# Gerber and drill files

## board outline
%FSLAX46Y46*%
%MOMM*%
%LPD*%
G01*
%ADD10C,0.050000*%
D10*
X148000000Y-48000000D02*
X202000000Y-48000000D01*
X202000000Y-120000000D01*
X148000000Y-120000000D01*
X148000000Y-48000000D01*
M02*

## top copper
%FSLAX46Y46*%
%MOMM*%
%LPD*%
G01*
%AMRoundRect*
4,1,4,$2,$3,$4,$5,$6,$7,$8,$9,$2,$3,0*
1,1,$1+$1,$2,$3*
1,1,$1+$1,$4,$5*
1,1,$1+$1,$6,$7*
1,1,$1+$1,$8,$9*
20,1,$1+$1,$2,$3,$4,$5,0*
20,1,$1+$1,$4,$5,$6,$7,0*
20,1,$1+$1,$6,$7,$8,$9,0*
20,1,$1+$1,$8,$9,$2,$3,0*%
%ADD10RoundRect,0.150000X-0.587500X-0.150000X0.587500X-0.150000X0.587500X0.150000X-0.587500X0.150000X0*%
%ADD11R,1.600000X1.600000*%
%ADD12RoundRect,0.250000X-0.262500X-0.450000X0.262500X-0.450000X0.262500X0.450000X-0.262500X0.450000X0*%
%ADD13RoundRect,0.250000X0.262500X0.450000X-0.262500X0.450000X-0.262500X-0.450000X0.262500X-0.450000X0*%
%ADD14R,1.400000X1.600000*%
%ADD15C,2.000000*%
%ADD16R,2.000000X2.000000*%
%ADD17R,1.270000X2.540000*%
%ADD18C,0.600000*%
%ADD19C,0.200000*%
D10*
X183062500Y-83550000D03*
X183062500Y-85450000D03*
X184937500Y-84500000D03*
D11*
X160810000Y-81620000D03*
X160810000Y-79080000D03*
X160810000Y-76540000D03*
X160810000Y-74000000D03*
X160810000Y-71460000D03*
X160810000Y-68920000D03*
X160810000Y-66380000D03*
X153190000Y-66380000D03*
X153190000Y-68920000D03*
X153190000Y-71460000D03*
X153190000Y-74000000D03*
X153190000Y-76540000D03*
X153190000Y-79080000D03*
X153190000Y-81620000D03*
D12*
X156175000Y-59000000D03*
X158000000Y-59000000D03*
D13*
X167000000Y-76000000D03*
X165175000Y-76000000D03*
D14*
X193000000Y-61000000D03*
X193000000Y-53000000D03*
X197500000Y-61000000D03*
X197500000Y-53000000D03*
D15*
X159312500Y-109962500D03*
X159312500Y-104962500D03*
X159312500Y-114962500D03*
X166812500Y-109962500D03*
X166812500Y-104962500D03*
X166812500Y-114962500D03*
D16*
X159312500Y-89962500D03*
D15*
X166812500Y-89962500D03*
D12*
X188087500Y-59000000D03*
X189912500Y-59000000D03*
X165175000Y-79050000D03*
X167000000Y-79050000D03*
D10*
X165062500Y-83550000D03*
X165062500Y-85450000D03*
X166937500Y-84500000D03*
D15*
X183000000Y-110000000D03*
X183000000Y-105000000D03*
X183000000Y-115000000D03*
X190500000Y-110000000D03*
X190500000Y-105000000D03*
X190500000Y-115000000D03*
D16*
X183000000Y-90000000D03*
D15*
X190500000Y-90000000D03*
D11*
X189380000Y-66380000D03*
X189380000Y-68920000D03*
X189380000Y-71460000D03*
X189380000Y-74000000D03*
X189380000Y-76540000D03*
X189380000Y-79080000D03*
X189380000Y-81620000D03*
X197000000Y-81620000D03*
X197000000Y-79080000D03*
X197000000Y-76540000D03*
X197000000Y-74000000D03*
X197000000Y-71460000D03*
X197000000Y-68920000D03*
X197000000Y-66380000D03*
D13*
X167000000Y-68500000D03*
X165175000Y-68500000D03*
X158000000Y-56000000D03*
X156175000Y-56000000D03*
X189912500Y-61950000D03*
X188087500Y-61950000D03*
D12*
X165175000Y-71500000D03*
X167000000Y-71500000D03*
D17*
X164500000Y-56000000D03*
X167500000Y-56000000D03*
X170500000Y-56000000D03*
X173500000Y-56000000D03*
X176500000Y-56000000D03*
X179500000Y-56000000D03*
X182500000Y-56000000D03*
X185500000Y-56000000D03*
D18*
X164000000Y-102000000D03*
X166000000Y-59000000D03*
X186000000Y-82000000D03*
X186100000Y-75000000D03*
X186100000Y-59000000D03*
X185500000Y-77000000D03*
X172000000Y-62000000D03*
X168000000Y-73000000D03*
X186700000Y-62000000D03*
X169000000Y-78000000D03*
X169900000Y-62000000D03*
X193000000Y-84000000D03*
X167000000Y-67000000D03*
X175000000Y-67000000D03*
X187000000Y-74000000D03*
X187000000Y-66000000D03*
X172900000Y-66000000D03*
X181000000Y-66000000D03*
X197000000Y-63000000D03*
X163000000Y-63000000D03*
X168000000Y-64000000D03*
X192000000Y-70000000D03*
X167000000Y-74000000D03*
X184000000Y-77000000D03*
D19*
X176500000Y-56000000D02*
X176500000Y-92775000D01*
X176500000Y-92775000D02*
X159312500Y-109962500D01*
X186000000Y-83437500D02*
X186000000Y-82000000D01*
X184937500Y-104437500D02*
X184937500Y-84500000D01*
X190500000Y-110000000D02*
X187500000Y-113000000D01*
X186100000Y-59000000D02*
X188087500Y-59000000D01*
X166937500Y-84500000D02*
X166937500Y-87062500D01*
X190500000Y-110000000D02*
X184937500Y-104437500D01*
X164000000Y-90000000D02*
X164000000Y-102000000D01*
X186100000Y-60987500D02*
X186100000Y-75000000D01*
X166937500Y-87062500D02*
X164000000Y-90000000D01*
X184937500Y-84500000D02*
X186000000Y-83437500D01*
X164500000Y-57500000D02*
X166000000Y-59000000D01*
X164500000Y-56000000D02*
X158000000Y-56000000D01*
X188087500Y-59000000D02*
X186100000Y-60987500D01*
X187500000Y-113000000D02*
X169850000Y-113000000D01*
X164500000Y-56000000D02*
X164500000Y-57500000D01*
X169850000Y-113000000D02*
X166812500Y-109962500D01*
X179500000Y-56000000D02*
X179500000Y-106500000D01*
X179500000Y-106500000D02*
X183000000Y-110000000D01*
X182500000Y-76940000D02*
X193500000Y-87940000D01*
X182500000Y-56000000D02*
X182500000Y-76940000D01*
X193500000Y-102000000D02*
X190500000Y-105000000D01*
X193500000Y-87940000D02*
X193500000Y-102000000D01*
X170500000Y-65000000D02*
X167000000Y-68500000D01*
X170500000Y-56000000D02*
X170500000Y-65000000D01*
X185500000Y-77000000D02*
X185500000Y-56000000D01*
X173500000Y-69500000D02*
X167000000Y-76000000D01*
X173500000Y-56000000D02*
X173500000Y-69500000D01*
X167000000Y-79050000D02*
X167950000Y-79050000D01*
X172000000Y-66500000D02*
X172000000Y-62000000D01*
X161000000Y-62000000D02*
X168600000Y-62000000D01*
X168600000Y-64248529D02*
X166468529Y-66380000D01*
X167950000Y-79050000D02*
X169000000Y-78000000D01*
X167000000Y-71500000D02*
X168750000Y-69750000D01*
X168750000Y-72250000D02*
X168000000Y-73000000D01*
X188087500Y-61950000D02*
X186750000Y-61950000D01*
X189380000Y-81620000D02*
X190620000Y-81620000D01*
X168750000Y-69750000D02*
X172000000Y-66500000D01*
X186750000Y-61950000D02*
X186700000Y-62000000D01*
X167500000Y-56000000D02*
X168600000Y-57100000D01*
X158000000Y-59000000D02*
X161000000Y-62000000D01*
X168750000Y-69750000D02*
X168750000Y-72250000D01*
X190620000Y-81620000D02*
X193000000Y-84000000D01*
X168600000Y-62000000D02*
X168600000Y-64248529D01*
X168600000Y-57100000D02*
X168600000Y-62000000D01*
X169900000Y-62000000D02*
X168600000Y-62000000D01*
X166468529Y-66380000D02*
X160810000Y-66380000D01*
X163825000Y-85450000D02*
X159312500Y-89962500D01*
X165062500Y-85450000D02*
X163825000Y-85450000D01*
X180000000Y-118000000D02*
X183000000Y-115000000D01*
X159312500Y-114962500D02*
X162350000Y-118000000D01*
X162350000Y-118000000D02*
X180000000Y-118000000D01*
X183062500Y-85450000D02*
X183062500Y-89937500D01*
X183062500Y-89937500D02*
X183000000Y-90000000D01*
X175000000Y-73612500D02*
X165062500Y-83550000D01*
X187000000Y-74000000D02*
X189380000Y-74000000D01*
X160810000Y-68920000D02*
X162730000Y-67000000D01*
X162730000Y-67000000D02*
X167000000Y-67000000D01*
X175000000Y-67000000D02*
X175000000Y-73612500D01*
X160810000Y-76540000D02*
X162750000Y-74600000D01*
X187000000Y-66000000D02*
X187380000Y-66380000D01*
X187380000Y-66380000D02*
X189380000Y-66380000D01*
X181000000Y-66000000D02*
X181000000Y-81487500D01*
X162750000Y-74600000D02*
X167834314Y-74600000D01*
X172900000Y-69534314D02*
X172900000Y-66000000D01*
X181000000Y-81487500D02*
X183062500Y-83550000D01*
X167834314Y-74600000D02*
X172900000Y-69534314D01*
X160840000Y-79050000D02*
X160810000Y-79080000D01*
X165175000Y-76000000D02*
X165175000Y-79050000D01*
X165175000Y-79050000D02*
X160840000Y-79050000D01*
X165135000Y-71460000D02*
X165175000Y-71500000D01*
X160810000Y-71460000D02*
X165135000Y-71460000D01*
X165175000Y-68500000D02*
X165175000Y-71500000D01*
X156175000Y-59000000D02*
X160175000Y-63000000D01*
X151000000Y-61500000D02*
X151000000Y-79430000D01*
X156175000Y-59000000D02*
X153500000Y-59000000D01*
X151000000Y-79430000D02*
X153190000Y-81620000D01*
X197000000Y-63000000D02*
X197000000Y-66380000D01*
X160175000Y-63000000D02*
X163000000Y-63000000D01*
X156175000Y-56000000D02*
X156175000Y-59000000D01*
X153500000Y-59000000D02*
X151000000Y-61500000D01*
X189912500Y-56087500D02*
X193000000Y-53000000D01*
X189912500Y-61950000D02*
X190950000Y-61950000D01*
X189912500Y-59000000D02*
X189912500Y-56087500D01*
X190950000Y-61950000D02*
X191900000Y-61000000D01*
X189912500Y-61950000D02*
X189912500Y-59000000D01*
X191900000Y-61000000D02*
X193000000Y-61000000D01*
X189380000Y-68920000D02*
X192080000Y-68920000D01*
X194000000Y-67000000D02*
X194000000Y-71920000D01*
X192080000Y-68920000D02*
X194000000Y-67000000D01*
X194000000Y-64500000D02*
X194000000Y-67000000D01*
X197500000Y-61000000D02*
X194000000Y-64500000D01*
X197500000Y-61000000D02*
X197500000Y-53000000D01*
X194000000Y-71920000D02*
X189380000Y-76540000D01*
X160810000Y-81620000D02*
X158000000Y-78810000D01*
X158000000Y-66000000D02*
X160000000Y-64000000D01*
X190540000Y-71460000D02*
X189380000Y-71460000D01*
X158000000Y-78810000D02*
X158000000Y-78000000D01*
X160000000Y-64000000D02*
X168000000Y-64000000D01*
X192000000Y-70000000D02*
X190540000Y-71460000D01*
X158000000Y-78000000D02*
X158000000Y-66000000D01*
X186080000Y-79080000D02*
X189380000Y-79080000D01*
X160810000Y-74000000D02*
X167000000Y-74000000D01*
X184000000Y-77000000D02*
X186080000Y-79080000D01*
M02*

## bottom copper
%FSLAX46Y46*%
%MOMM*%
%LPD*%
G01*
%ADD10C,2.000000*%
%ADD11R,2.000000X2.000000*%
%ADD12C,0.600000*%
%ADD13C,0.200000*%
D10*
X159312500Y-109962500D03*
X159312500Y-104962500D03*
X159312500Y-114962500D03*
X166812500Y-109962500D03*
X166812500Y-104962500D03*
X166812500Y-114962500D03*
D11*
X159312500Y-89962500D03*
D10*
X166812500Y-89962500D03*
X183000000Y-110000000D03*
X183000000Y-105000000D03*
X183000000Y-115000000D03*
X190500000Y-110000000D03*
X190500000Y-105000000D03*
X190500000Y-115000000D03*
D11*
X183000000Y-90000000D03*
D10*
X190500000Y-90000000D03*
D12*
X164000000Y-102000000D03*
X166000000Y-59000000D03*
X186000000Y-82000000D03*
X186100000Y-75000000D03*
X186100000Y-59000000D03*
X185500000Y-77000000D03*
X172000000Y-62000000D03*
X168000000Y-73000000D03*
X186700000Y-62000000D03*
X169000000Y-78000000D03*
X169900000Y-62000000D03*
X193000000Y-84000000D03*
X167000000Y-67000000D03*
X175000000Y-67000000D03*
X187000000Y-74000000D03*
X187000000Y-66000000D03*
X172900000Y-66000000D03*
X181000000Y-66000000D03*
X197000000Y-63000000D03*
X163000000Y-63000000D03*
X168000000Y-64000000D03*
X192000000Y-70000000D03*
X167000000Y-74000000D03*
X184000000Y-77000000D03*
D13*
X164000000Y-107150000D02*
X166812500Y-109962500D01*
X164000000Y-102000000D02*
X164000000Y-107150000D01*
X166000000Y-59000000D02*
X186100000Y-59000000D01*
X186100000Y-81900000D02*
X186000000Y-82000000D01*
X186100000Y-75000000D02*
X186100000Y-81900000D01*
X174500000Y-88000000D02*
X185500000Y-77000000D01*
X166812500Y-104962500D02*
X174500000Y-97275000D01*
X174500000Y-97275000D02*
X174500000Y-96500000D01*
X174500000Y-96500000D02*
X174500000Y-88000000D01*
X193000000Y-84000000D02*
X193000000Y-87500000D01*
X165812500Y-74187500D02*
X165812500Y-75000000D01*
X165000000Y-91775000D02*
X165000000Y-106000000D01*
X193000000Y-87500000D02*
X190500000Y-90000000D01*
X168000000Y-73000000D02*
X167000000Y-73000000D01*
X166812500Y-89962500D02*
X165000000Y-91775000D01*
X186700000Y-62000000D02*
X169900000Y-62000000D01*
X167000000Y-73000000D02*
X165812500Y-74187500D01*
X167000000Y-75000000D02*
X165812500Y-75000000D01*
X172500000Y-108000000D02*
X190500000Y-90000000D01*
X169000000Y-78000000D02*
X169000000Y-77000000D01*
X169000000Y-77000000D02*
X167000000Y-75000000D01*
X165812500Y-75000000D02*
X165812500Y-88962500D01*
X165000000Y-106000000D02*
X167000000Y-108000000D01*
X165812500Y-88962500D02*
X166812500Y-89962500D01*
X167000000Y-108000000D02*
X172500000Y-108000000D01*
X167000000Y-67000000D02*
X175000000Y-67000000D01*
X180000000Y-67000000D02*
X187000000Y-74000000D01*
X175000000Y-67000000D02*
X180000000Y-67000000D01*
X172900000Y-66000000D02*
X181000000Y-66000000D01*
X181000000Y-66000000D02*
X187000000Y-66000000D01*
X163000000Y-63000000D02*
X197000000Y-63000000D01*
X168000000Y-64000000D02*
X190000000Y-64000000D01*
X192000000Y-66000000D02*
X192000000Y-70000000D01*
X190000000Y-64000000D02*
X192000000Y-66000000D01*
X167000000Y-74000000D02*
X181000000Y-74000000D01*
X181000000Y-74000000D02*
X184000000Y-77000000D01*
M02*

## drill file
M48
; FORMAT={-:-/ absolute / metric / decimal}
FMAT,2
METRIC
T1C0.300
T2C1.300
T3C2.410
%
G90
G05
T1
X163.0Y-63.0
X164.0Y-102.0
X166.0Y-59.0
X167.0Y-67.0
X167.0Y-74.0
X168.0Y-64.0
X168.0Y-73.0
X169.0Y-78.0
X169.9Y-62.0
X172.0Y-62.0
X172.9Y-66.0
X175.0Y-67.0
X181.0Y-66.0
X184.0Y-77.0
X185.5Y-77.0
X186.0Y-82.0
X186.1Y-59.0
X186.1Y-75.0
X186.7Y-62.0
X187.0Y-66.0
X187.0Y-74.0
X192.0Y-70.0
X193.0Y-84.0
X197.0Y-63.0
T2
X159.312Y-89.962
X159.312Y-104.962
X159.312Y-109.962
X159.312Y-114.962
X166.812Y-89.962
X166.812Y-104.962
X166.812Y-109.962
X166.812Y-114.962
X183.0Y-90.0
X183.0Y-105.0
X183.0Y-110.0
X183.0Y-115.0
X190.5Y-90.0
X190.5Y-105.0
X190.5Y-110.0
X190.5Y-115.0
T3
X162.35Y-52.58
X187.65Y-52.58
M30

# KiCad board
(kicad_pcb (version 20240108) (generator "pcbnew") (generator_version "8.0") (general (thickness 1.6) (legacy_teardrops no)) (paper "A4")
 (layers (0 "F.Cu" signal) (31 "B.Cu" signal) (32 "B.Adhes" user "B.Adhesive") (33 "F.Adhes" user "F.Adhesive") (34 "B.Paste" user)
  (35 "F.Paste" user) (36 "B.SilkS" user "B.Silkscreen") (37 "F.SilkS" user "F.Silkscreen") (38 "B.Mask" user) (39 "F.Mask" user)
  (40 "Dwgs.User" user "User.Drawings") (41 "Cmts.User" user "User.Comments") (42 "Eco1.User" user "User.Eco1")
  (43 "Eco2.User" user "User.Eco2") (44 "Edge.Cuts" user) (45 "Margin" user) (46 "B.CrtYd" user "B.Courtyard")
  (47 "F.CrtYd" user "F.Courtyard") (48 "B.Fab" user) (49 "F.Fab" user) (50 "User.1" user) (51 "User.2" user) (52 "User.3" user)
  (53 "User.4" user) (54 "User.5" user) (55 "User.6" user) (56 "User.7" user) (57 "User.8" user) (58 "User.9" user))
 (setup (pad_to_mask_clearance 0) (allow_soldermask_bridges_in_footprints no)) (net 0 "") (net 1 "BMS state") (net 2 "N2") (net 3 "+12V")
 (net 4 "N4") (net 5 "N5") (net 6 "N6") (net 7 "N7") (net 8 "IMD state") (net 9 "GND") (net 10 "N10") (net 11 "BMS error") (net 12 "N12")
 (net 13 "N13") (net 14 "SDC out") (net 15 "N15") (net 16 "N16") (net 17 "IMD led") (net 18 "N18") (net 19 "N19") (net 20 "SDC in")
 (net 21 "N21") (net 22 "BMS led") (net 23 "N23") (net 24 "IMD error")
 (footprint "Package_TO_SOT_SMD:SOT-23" (layer "F.Cu") (at 184 84.5)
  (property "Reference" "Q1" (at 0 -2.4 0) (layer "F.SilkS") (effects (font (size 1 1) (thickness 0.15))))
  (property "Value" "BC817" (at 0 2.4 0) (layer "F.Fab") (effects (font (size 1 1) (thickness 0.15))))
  (pad "1" smd roundrect (at -0.9375 -0.95) (size 1.475 0.6) (layers "F.Cu" "F.Paste" "F.Mask") (roundrect_rratio 0.25) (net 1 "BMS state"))
  (pad "2" smd roundrect (at -0.9375 0.95) (size 1.475 0.6) (layers "F.Cu" "F.Paste" "F.Mask") (roundrect_rratio 0.25) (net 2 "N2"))
  (pad "3" smd roundrect (at 0.9375 0) (size 1.475 0.6) (layers "F.Cu" "F.Paste" "F.Mask") (roundrect_rratio 0.25) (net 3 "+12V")))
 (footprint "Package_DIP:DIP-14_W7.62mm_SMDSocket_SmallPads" (layer "F.Cu") (at 157 74 180)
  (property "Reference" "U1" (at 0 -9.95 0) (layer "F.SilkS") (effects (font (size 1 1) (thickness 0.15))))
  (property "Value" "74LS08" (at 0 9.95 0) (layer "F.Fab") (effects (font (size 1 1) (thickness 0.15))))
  (pad "1" smd rect (at -3.81 -7.62 180) (size 1.6 1.6) (layers "F.Cu" "F.Paste" "F.Mask") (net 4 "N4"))
  (pad "2" smd rect (at -3.81 -5.08 180) (size 1.6 1.6) (layers "F.Cu" "F.Paste" "F.Mask") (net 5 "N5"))
  (pad "3" smd rect (at -3.81 -2.54 180) (size 1.6 1.6) (layers "F.Cu" "F.Paste" "F.Mask") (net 1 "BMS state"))
  (pad "4" smd rect (at -3.81 0 180) (size 1.6 1.6) (layers "F.Cu" "F.Paste" "F.Mask") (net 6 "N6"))
  (pad "5" smd rect (at -3.81 2.54 180) (size 1.6 1.6) (layers "F.Cu" "F.Paste" "F.Mask") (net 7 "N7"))
  (pad "6" smd rect (at -3.81 5.08 180) (size 1.6 1.6) (layers "F.Cu" "F.Paste" "F.Mask") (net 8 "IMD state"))
  (pad "7" smd rect (at -3.81 7.62 180) (size 1.6 1.6) (layers "F.Cu" "F.Paste" "F.Mask") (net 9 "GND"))
  (pad "8" smd rect (at 3.81 7.62 180) (size 1.6 1.6) (layers "F.Cu" "F.Paste" "F.Mask"))
  (pad "9" smd rect (at 3.81 5.08 180) (size 1.6 1.6) (layers "F.Cu" "F.Paste" "F.Mask"))
  (pad "10" smd rect (at 3.81 2.54 180) (size 1.6 1.6) (layers "F.Cu" "F.Paste" "F.Mask"))
  (pad "11" smd rect (at 3.81 0 180) (size 1.6 1.6) (layers "F.Cu" "F.Paste" "F.Mask"))
  (pad "12" smd rect (at 3.81 -2.54 180) (size 1.6 1.6) (layers "F.Cu" "F.Paste" "F.Mask"))
  (pad "13" smd rect (at 3.81 -5.08 180) (size 1.6 1.6) (layers "F.Cu" "F.Paste" "F.Mask"))
  (pad "14" smd rect (at 3.81 -7.62 180) (size 1.6 1.6) (layers "F.Cu" "F.Paste" "F.Mask") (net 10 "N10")))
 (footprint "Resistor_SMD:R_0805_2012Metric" (layer "F.Cu") (at 157.0875 59)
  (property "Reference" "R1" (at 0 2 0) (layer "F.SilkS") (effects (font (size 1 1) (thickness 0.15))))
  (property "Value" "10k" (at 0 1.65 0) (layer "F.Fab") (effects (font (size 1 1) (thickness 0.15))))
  (pad "1" smd roundrect (at -0.9125 0) (size 1.025 1.4) (layers "F.Cu" "F.Paste" "F.Mask") (roundrect_rratio 0.243902) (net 10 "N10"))
  (pad "2" smd roundrect (at 0.9125 0) (size 1.025 1.4) (layers "F.Cu" "F.Paste" "F.Mask") (roundrect_rratio 0.243902) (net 9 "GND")))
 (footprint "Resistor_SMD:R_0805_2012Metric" (layer "F.Cu") (at 166.0875 76 180)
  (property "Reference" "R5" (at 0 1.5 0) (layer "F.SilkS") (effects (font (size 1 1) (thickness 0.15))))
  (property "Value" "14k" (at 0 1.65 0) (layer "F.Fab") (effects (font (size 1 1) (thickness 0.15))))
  (pad "1" smd roundrect (at -0.9125 0 180) (size 1.025 1.4) (layers "F.Cu" "F.Paste" "F.Mask") (roundrect_rratio 0.243902)
   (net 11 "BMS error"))
  (pad "2" smd roundrect (at 0.9125 0 180) (size 1.025 1.4) (layers "F.Cu" "F.Paste" "F.Mask") (roundrect_rratio 0.243902) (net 5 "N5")))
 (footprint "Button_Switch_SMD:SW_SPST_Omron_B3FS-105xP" (layer "F.Cu") (at 195.25 57 90)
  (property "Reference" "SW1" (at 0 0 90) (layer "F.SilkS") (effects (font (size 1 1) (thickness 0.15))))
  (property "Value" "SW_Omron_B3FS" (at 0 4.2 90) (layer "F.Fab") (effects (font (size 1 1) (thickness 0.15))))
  (pad "1" smd rect (at -4 -2.25 270) (size 1.6 1.4) (layers "F.Cu" "F.Paste" "F.Mask") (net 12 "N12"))
  (pad "1" smd rect (at 4 -2.25 270) (size 1.6 1.4) (layers "F.Cu" "F.Paste" "F.Mask") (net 12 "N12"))
  (pad "2" smd rect (at -4 2.25 270) (size 1.6 1.4) (layers "F.Cu" "F.Paste" "F.Mask") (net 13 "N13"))
  (pad "2" smd rect (at 4 2.25 270) (size 1.6 1.4) (layers "F.Cu" "F.Paste" "F.Mask") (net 13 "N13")))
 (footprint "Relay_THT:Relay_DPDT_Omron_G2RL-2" (layer "F.Cu") (at 159.3125 89.9625)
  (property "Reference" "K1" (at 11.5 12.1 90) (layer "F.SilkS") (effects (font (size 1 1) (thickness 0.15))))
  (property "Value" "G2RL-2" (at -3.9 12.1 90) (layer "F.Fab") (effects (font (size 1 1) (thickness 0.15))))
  (pad "11" thru_hole circle (at 0 20) (size 2 2) (drill 1.3) (layers "*.Cu" "*.Mask") (remove_unused_layers no) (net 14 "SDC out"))
  (pad "12" thru_hole circle (at 0 15) (size 2 2) (drill 1.3) (layers "*.Cu" "*.Mask") (remove_unused_layers no) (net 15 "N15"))
  (pad "14" thru_hole circle (at 0 25) (size 2 2) (drill 1.3) (layers "*.Cu" "*.Mask") (remove_unused_layers no) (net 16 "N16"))
  (pad "21" thru_hole circle (at 7.5 20) (size 2 2) (drill 1.3) (layers "*.Cu" "*.Mask") (remove_unused_layers no) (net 3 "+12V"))
  (pad "22" thru_hole circle (at 7.5 15) (size 2 2) (drill 1.3) (layers "*.Cu" "*.Mask") (remove_unused_layers no) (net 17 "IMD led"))
  (pad "24" thru_hole circle (at 7.5 25) (size 2 2) (drill 1.3) (layers "*.Cu" "*.Mask") (remove_unused_layers no) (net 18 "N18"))
  (pad "A1" thru_hole rect (at 0 0) (size 2 2) (drill 1.3) (layers "*.Cu" "*.Mask") (remove_unused_layers no) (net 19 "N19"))
  (pad "A2" thru_hole circle (at 7.5 0) (size 2 2) (drill 1.3) (layers "*.Cu" "*.Mask") (remove_unused_layers no) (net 9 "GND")))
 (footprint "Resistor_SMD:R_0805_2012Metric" (layer "F.Cu") (at 189 59)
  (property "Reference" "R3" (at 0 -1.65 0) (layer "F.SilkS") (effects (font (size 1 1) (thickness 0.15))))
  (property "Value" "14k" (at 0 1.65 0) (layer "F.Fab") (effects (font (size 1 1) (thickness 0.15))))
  (pad "1" smd roundrect (at -0.9125 0) (size 1.025 1.4) (layers "F.Cu" "F.Paste" "F.Mask") (roundrect_rratio 0.243902) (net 3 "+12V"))
  (pad "2" smd roundrect (at 0.9125 0) (size 1.025 1.4) (layers "F.Cu" "F.Paste" "F.Mask") (roundrect_rratio 0.243902) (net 12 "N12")))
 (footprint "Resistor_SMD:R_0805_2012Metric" (layer "F.Cu") (at 166.0875 79.05)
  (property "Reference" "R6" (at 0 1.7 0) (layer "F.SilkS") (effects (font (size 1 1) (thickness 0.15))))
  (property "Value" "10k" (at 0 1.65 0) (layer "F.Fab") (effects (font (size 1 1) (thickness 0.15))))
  (pad "1" smd roundrect (at -0.9125 0) (size 1.025 1.4) (layers "F.Cu" "F.Paste" "F.Mask") (roundrect_rratio 0.243902) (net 5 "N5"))
  (pad "2" smd roundrect (at 0.9125 0) (size 1.025 1.4) (layers "F.Cu" "F.Paste" "F.Mask") (roundrect_rratio 0.243902) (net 9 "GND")))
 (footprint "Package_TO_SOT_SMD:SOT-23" (layer "F.Cu") (at 166 84.5)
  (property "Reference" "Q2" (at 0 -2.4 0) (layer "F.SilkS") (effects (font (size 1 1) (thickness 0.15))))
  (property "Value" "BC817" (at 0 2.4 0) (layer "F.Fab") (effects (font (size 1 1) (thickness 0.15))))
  (pad "1" smd roundrect (at -0.9375 -0.95) (size 1.475 0.6) (layers "F.Cu" "F.Paste" "F.Mask") (roundrect_rratio 0.25) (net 8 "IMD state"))
  (pad "2" smd roundrect (at -0.9375 0.95) (size 1.475 0.6) (layers "F.Cu" "F.Paste" "F.Mask") (roundrect_rratio 0.25) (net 19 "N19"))
  (pad "3" smd roundrect (at 0.9375 0) (size 1.475 0.6) (layers "F.Cu" "F.Paste" "F.Mask") (roundrect_rratio 0.25) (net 3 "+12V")))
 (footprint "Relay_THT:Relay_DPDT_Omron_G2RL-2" (layer "F.Cu") (at 183 90)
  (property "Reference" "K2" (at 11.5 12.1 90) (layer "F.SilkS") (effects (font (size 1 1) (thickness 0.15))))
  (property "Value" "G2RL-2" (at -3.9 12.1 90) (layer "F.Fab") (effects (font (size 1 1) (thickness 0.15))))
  (pad "11" thru_hole circle (at 0 20) (size 2 2) (drill 1.3) (layers "*.Cu" "*.Mask") (remove_unused_layers no) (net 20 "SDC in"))
  (pad "12" thru_hole circle (at 0 15) (size 2 2) (drill 1.3) (layers "*.Cu" "*.Mask") (remove_unused_layers no) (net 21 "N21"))
  (pad "14" thru_hole circle (at 0 25) (size 2 2) (drill 1.3) (layers "*.Cu" "*.Mask") (remove_unused_layers no) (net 16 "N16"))
  (pad "21" thru_hole circle (at 7.5 20) (size 2 2) (drill 1.3) (layers "*.Cu" "*.Mask") (remove_unused_layers no) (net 3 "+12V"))
  (pad "22" thru_hole circle (at 7.5 15) (size 2 2) (drill 1.3) (layers "*.Cu" "*.Mask") (remove_unused_layers no) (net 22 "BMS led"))
  (pad "24" thru_hole circle (at 7.5 25) (size 2 2) (drill 1.3) (layers "*.Cu" "*.Mask") (remove_unused_layers no) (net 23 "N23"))
  (pad "A1" thru_hole rect (at 0 0) (size 2 2) (drill 1.3) (layers "*.Cu" "*.Mask") (remove_unused_layers no) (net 2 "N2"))
  (pad "A2" thru_hole circle (at 7.5 0) (size 2 2) (drill 1.3) (layers "*.Cu" "*.Mask") (remove_unused_layers no) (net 9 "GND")))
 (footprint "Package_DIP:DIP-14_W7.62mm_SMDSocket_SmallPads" (layer "F.Cu") (at 193.19 74)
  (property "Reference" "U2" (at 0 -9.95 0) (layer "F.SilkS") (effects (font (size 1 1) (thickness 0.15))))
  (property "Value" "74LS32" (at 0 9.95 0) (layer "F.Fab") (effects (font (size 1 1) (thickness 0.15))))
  (pad "1" smd rect (at -3.81 -7.62) (size 1.6 1.6) (layers "F.Cu" "F.Paste" "F.Mask") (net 1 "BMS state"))
  (pad "2" smd rect (at -3.81 -5.08) (size 1.6 1.6) (layers "F.Cu" "F.Paste" "F.Mask") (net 13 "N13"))
  (pad "3" smd rect (at -3.81 -2.54) (size 1.6 1.6) (layers "F.Cu" "F.Paste" "F.Mask") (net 4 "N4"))
  (pad "4" smd rect (at -3.81 0) (size 1.6 1.6) (layers "F.Cu" "F.Paste" "F.Mask") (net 8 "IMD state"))
  (pad "5" smd rect (at -3.81 2.54) (size 1.6 1.6) (layers "F.Cu" "F.Paste" "F.Mask") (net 13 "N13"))
  (pad "6" smd rect (at -3.81 5.08) (size 1.6 1.6) (layers "F.Cu" "F.Paste" "F.Mask") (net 6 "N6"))
  (pad "7" smd rect (at -3.81 7.62) (size 1.6 1.6) (layers "F.Cu" "F.Paste" "F.Mask") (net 9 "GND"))
  (pad "8" smd rect (at 3.81 7.62) (size 1.6 1.6) (layers "F.Cu" "F.Paste" "F.Mask"))
  (pad "9" smd rect (at 3.81 5.08) (size 1.6 1.6) (layers "F.Cu" "F.Paste" "F.Mask"))
  (pad "10" smd rect (at 3.81 2.54) (size 1.6 1.6) (layers "F.Cu" "F.Paste" "F.Mask"))
  (pad "11" smd rect (at 3.81 0) (size 1.6 1.6) (layers "F.Cu" "F.Paste" "F.Mask"))
  (pad "12" smd rect (at 3.81 -2.54) (size 1.6 1.6) (layers "F.Cu" "F.Paste" "F.Mask"))
  (pad "13" smd rect (at 3.81 -5.08) (size 1.6 1.6) (layers "F.Cu" "F.Paste" "F.Mask"))
  (pad "14" smd rect (at 3.81 -7.62) (size 1.6 1.6) (layers "F.Cu" "F.Paste" "F.Mask") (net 10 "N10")))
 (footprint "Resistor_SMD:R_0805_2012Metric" (layer "F.Cu") (at 166.0875 68.5 180)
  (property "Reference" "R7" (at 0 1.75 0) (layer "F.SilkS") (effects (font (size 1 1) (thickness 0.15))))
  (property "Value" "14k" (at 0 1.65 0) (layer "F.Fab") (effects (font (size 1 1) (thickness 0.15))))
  (pad "1" smd roundrect (at -0.9125 0 180) (size 1.025 1.4) (layers "F.Cu" "F.Paste" "F.Mask") (roundrect_rratio 0.243902)
   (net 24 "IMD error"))
  (pad "2" smd roundrect (at 0.9125 0 180) (size 1.025 1.4) (layers "F.Cu" "F.Paste" "F.Mask") (roundrect_rratio 0.243902) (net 7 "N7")))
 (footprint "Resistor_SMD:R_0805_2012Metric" (layer "F.Cu") (at 157.0875 56 180)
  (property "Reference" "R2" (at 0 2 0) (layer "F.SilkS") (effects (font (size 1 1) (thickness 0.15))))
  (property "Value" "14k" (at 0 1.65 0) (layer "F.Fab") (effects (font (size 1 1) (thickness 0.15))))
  (pad "1" smd roundrect (at -0.9125 0 180) (size 1.025 1.4) (layers "F.Cu" "F.Paste" "F.Mask") (roundrect_rratio 0.243902) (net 3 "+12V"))
  (pad "2" smd roundrect (at 0.9125 0 180) (size 1.025 1.4) (layers "F.Cu" "F.Paste" "F.Mask") (roundrect_rratio 0.243902) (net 10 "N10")))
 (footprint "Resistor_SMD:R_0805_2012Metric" (layer "F.Cu") (at 189 61.95 180)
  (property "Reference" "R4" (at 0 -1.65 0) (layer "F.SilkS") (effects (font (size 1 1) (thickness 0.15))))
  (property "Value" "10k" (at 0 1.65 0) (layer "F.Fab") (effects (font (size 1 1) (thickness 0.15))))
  (pad "1" smd roundrect (at -0.9125 0 180) (size 1.025 1.4) (layers "F.Cu" "F.Paste" "F.Mask") (roundrect_rratio 0.243902) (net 12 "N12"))
  (pad "2" smd roundrect (at 0.9125 0 180) (size 1.025 1.4) (layers "F.Cu" "F.Paste" "F.Mask") (roundrect_rratio 0.243902) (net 9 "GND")))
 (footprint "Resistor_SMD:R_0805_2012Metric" (layer "F.Cu") (at 166.0875 71.5)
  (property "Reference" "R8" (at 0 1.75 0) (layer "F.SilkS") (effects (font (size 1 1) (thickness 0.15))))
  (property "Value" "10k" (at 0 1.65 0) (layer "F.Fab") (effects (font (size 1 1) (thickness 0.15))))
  (pad "1" smd roundrect (at -0.9125 0) (size 1.025 1.4) (layers "F.Cu" "F.Paste" "F.Mask") (roundrect_rratio 0.243902) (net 7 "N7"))
  (pad "2" smd roundrect (at 0.9125 0) (size 1.025 1.4) (layers "F.Cu" "F.Paste" "F.Mask") (roundrect_rratio 0.243902) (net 9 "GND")))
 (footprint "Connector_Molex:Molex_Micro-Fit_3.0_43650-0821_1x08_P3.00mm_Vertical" (layer "F.Cu") (at 175 52.865)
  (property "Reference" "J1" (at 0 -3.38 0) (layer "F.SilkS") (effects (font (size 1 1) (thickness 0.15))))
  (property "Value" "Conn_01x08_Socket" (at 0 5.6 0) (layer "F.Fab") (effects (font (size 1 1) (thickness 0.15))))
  (pad "" np_thru_hole circle (at -12.65 -0.285) (size 2.41 2.41) (drill 2.41) (layers "*.Cu" "*.Mask"))
  (pad "" np_thru_hole circle (at 12.65 -0.285) (size 2.41 2.41) (drill 2.41) (layers "*.Cu" "*.Mask"))
  (pad "1" smd rect (at -10.5 3.135) (size 1.27 2.54) (layers "F.Cu" "F.Paste" "F.Mask") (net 3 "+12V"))
  (pad "2" smd rect (at -7.5 3.135) (size 1.27 2.54) (layers "F.Cu" "F.Paste" "F.Mask") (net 9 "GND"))
  (pad "3" smd rect (at -4.5 3.135) (size 1.27 2.54) (layers "F.Cu" "F.Paste" "F.Mask") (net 24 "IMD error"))
  (pad "4" smd rect (at -1.5 3.135) (size 1.27 2.54) (layers "F.Cu" "F.Paste" "F.Mask") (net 11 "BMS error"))
  (pad "5" smd rect (at 1.5 3.135) (size 1.27 2.54) (layers "F.Cu" "F.Paste" "F.Mask") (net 14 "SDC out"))
  (pad "6" smd rect (at 4.5 3.135) (size 1.27 2.54) (layers "F.Cu" "F.Paste" "F.Mask") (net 20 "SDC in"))
  (pad "7" smd rect (at 7.5 3.135) (size 1.27 2.54) (layers "F.Cu" "F.Paste" "F.Mask") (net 22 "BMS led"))
  (pad "8" smd rect (at 10.5 3.135) (size 1.27 2.54) (layers "F.Cu" "F.Paste" "F.Mask") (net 17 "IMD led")))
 (gr_rect (start 148 48) (end 202 120) (stroke (width 0.05) (type default)) (fill none) (layer "Edge.Cuts"))
 (segment (start 176.5 56) (end 176.5 92.775) (width 0.2) (layer "F.Cu") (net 14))
 (segment (start 176.5 92.775) (end 159.3125 109.9625) (width 0.2) (layer "F.Cu") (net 14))
 (segment (start 186 83.4375) (end 186 82) (width 0.2) (layer "F.Cu") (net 3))
 (segment (start 184.9375 104.4375) (end 184.9375 84.5) (width 0.2) (layer "F.Cu") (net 3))
 (segment (start 190.5 110) (end 187.5 113) (width 0.2) (layer "F.Cu") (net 3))
 (segment (start 186.1 59) (end 188.0875 59) (width 0.2) (layer "F.Cu") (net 3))
 (segment (start 166.9375 84.5) (end 166.9375 87.0625) (width 0.2) (layer "F.Cu") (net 3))
 (segment (start 190.5 110) (end 184.9375 104.4375) (width 0.2) (layer "F.Cu") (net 3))
 (segment (start 164 90) (end 164 102) (width 0.2) (layer "F.Cu") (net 3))
 (segment (start 186.1 60.9875) (end 186.1 75) (width 0.2) (layer "F.Cu") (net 3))
 (segment (start 166.9375 87.0625) (end 164 90) (width 0.2) (layer "F.Cu") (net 3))
 (segment (start 184.9375 84.5) (end 186 83.4375) (width 0.2) (layer "F.Cu") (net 3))
 (segment (start 164.5 57.5) (end 166 59) (width 0.2) (layer "F.Cu") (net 3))
 (segment (start 164.5 56) (end 158 56) (width 0.2) (layer "F.Cu") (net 3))
 (segment (start 188.0875 59) (end 186.1 60.9875) (width 0.2) (layer "F.Cu") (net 3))
 (segment (start 187.5 113) (end 169.85 113) (width 0.2) (layer "F.Cu") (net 3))
 (segment (start 164.5 56) (end 164.5 57.5) (width 0.2) (layer "F.Cu") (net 3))
 (segment (start 169.85 113) (end 166.8125 109.9625) (width 0.2) (layer "F.Cu") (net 3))
 (via (at 164 102) (size 0.6) (drill 0.3) (layers "F.Cu" "B.Cu") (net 3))
 (via (at 166 59) (size 0.6) (drill 0.3) (layers "F.Cu" "B.Cu") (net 3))
 (via (at 186 82) (size 0.6) (drill 0.3) (layers "F.Cu" "B.Cu") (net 3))
 (via (at 186.1 75) (size 0.6) (drill 0.3) (layers "F.Cu" "B.Cu") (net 3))
 (via (at 186.1 59) (size 0.6) (drill 0.3) (layers "F.Cu" "B.Cu") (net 3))
 (segment (start 164 107.15) (end 166.8125 109.9625) (width 0.2) (layer "B.Cu") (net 3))
 (segment (start 164 102) (end 164 107.15) (width 0.2) (layer "B.Cu") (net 3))
 (segment (start 166 59) (end 186.1 59) (width 0.2) (layer "B.Cu") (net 3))
 (segment (start 186.1 81.9) (end 186 82) (width 0.2) (layer "B.Cu") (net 3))
 (segment (start 186.1 75) (end 186.1 81.9) (width 0.2) (layer "B.Cu") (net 3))
 (segment (start 179.5 56) (end 179.5 106.5) (width 0.2) (layer "F.Cu") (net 20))
 (segment (start 179.5 106.5) (end 183 110) (width 0.2) (layer "F.Cu") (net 20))
 (segment (start 182.5 76.94) (end 193.5 87.94) (width 0.2) (layer "F.Cu") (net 22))
 (segment (start 182.5 56) (end 182.5 76.94) (width 0.2) (layer "F.Cu") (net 22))
 (segment (start 193.5 102) (end 190.5 105) (width 0.2) (layer "F.Cu") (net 22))
 (segment (start 193.5 87.94) (end 193.5 102) (width 0.2) (layer "F.Cu") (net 22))
 (segment (start 170.5 65) (end 167 68.5) (width 0.2) (layer "F.Cu") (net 24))
 (segment (start 170.5 56) (end 170.5 65) (width 0.2) (layer "F.Cu") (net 24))
 (segment (start 185.5 77) (end 185.5 56) (width 0.2) (layer "F.Cu") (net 17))
 (via (at 185.5 77) (size 0.6) (drill 0.3) (layers "F.Cu" "B.Cu") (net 17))
 (segment (start 174.5 88) (end 185.5 77) (width 0.2) (layer "B.Cu") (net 17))
 (segment (start 166.8125 104.9625) (end 174.5 97.275) (width 0.2) (layer "B.Cu") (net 17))
 (segment (start 174.5 97.275) (end 174.5 96.5) (width 0.2) (layer "B.Cu") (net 17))
 (segment (start 174.5 96.5) (end 174.5 88) (width 0.2) (layer "B.Cu") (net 17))
 (segment (start 173.5 69.5) (end 167 76) (width 0.2) (layer "F.Cu") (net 11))
 (segment (start 173.5 56) (end 173.5 69.5) (width 0.2) (layer "F.Cu") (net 11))
 (segment (start 167 79.05) (end 167.95 79.05) (width 0.2) (layer "F.Cu") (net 9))
 (segment (start 172 66.5) (end 172 62) (width 0.2) (layer "F.Cu") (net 9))
 (segment (start 161 62) (end 168.6 62) (width 0.2) (layer "F.Cu") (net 9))
 (segment (start 168.6 64.248529) (end 166.468529 66.38) (width 0.2) (layer "F.Cu") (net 9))
 (segment (start 167.95 79.05) (end 169 78) (width 0.2) (layer "F.Cu") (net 9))
 (segment (start 167 71.5) (end 168.75 69.75) (width 0.2) (layer "F.Cu") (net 9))
 (segment (start 168.75 72.25) (end 168 73) (width 0.2) (layer "F.Cu") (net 9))
 (segment (start 188.0875 61.95) (end 186.75 61.95) (width 0.2) (layer "F.Cu") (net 9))
 (segment (start 189.38 81.62) (end 190.62 81.62) (width 0.2) (layer "F.Cu") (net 9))
 (segment (start 168.75 69.75) (end 172 66.5) (width 0.2) (layer "F.Cu") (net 9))
 (segment (start 186.75 61.95) (end 186.7 62) (width 0.2) (layer "F.Cu") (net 9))
 (segment (start 167.5 56) (end 168.6 57.1) (width 0.2) (layer "F.Cu") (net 9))
 (segment (start 158 59) (end 161 62) (width 0.2) (layer "F.Cu") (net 9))
 (segment (start 168.75 69.75) (end 168.75 72.25) (width 0.2) (layer "F.Cu") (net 9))
 (segment (start 190.62 81.62) (end 193 84) (width 0.2) (layer "F.Cu") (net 9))
 (segment (start 168.6 62) (end 168.6 64.248529) (width 0.2) (layer "F.Cu") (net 9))
 (segment (start 168.6 57.1) (end 168.6 62) (width 0.2) (layer "F.Cu") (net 9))
 (segment (start 169.9 62) (end 168.6 62) (width 0.2) (layer "F.Cu") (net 9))
 (segment (start 166.468529 66.38) (end 160.81 66.38) (width 0.2) (layer "F.Cu") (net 9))
 (via (at 172 62) (size 0.6) (drill 0.3) (layers "F.Cu" "B.Cu") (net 9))
 (via (at 168 73) (size 0.6) (drill 0.3) (layers "F.Cu" "B.Cu") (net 9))
 (via (at 186.7 62) (size 0.6) (drill 0.3) (layers "F.Cu" "B.Cu") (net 9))
 (via (at 169 78) (size 0.6) (drill 0.3) (layers "F.Cu" "B.Cu") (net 9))
 (via (at 169.9 62) (size 0.6) (drill 0.3) (layers "F.Cu" "B.Cu") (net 9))
 (via (at 193 84) (size 0.6) (drill 0.3) (layers "F.Cu" "B.Cu") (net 9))
 (segment (start 193 84) (end 193 87.5) (width 0.2) (layer "B.Cu") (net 9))
 (segment (start 165.8125 74.1875) (end 165.8125 75) (width 0.2) (layer "B.Cu") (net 9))
 (segment (start 165 91.775) (end 165 106) (width 0.2) (layer "B.Cu") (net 9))
 (segment (start 193 87.5) (end 190.5 90) (width 0.2) (layer "B.Cu") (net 9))
 (segment (start 168 73) (end 167 73) (width 0.2) (layer "B.Cu") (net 9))
 (segment (start 166.8125 89.9625) (end 165 91.775) (width 0.2) (layer "B.Cu") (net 9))
 (segment (start 186.7 62) (end 169.9 62) (width 0.2) (layer "B.Cu") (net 9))
 (segment (start 167 73) (end 165.8125 74.1875) (width 0.2) (layer "B.Cu") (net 9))
 (segment (start 167 75) (end 165.8125 75) (width 0.2) (layer "B.Cu") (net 9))
 (segment (start 172.5 108) (end 190.5 90) (width 0.2) (layer "B.Cu") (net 9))
 (segment (start 169 78) (end 169 77) (width 0.2) (layer "B.Cu") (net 9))
 (segment (start 169 77) (end 167 75) (width 0.2) (layer "B.Cu") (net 9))
 (segment (start 165.8125 75) (end 165.8125 88.9625) (width 0.2) (layer "B.Cu") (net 9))
 (segment (start 165 106) (end 167 108) (width 0.2) (layer "B.Cu") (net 9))
 (segment (start 165.8125 88.9625) (end 166.8125 89.9625) (width 0.2) (layer "B.Cu") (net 9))
 (segment (start 167 108) (end 172.5 108) (width 0.2) (layer "B.Cu") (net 9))
 (segment (start 163.825 85.45) (end 159.3125 89.9625) (width 0.2) (layer "F.Cu") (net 19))
 (segment (start 165.0625 85.45) (end 163.825 85.45) (width 0.2) (layer "F.Cu") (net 19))
 (segment (start 180 118) (end 183 115) (width 0.2) (layer "F.Cu") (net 16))
 (segment (start 159.3125 114.9625) (end 162.35 118) (width 0.2) (layer "F.Cu") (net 16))
 (segment (start 162.35 118) (end 180 118) (width 0.2) (layer "F.Cu") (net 16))
 (segment (start 183.0625 85.45) (end 183.0625 89.9375) (width 0.2) (layer "F.Cu") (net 2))
 (segment (start 183.0625 89.9375) (end 183 90) (width 0.2) (layer "F.Cu") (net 2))
 (segment (start 175 73.6125) (end 165.0625 83.55) (width 0.2) (layer "F.Cu") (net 8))
 (segment (start 187 74) (end 189.38 74) (width 0.2) (layer "F.Cu") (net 8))
 (segment (start 160.81 68.92) (end 162.73 67) (width 0.2) (layer "F.Cu") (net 8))
 (segment (start 162.73 67) (end 167 67) (width 0.2) (layer "F.Cu") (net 8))
 (segment (start 175 67) (end 175 73.6125) (width 0.2) (layer "F.Cu") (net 8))
 (via (at 167 67) (size 0.6) (drill 0.3) (layers "F.Cu" "B.Cu") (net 8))
 (via (at 175 67) (size 0.6) (drill 0.3) (layers "F.Cu" "B.Cu") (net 8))
 (via (at 187 74) (size 0.6) (drill 0.3) (layers "F.Cu" "B.Cu") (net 8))
 (segment (start 167 67) (end 175 67) (width 0.2) (layer "B.Cu") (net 8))
 (segment (start 180 67) (end 187 74) (width 0.2) (layer "B.Cu") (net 8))
 (segment (start 175 67) (end 180 67) (width 0.2) (layer "B.Cu") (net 8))
 (segment (start 160.81 76.54) (end 162.75 74.6) (width 0.2) (layer "F.Cu") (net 1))
 (segment (start 187 66) (end 187.38 66.38) (width 0.2) (layer "F.Cu") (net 1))
 (segment (start 187.38 66.38) (end 189.38 66.38) (width 0.2) (layer "F.Cu") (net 1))
 (segment (start 181 66) (end 181 81.4875) (width 0.2) (layer "F.Cu") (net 1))
 (segment (start 162.75 74.6) (end 167.834314 74.6) (width 0.2) (layer "F.Cu") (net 1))
 (segment (start 172.9 69.534314) (end 172.9 66) (width 0.2) (layer "F.Cu") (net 1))
 (segment (start 181 81.4875) (end 183.0625 83.55) (width 0.2) (layer "F.Cu") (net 1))
 (segment (start 167.834314 74.6) (end 172.9 69.534314) (width 0.2) (layer "F.Cu") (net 1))
 (via (at 187 66) (size 0.6) (drill 0.3) (layers "F.Cu" "B.Cu") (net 1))
 (via (at 172.9 66) (size 0.6) (drill 0.3) (layers "F.Cu" "B.Cu") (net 1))
 (via (at 181 66) (size 0.6) (drill 0.3) (layers "F.Cu" "B.Cu") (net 1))
 (segment (start 172.9 66) (end 181 66) (width 0.2) (layer "B.Cu") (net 1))
 (segment (start 181 66) (end 187 66) (width 0.2) (layer "B.Cu") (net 1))
 (segment (start 160.84 79.05) (end 160.81 79.08) (width 0.2) (layer "F.Cu") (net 5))
 (segment (start 165.175 76) (end 165.175 79.05) (width 0.2) (layer "F.Cu") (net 5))
 (segment (start 165.175 79.05) (end 160.84 79.05) (width 0.2) (layer "F.Cu") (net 5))
 (segment (start 165.135 71.46) (end 165.175 71.5) (width 0.2) (layer "F.Cu") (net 7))
 (segment (start 160.81 71.46) (end 165.135 71.46) (width 0.2) (layer "F.Cu") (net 7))
 (segment (start 165.175 68.5) (end 165.175 71.5) (width 0.2) (layer "F.Cu") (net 7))
 (segment (start 156.175 59) (end 160.175 63) (width 0.2) (layer "F.Cu") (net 10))
 (segment (start 151 61.5) (end 151 79.43) (width 0.2) (layer "F.Cu") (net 10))
 (segment (start 156.175 59) (end 153.5 59) (width 0.2) (layer "F.Cu") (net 10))
 (segment (start 151 79.43) (end 153.19 81.62) (width 0.2) (layer "F.Cu") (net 10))
 (segment (start 197 63) (end 197 66.38) (width 0.2) (layer "F.Cu") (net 10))
 (segment (start 160.175 63) (end 163 63) (width 0.2) (layer "F.Cu") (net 10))
 (segment (start 156.175 56) (end 156.175 59) (width 0.2) (layer "F.Cu") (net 10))
 (segment (start 153.5 59) (end 151 61.5) (width 0.2) (layer "F.Cu") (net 10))
 (via (at 197 63) (size 0.6) (drill 0.3) (layers "F.Cu" "B.Cu") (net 10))
 (via (at 163 63) (size 0.6) (drill 0.3) (layers "F.Cu" "B.Cu") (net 10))
 (segment (start 163 63) (end 197 63) (width 0.2) (layer "B.Cu") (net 10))
 (segment (start 189.9125 56.0875) (end 193 53) (width 0.2) (layer "F.Cu") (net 12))
 (segment (start 189.9125 61.95) (end 190.95 61.95) (width 0.2) (layer "F.Cu") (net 12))
 (segment (start 189.9125 59) (end 189.9125 56.0875) (width 0.2) (layer "F.Cu") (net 12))
 (segment (start 190.95 61.95) (end 191.9 61) (width 0.2) (layer "F.Cu") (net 12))
 (segment (start 189.9125 61.95) (end 189.9125 59) (width 0.2) (layer "F.Cu") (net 12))
 (segment (start 191.9 61) (end 193 61) (width 0.2) (layer "F.Cu") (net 12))
 (segment (start 189.38 68.92) (end 192.08 68.92) (width 0.2) (layer "F.Cu") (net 13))
 (segment (start 194 67) (end 194 71.92) (width 0.2) (layer "F.Cu") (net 13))
 (segment (start 192.08 68.92) (end 194 67) (width 0.2) (layer "F.Cu") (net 13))
 (segment (start 194 64.5) (end 194 67) (width 0.2) (layer "F.Cu") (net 13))
 (segment (start 197.5 61) (end 194 64.5) (width 0.2) (layer "F.Cu") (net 13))
 (segment (start 197.5 61) (end 197.5 53) (width 0.2) (layer "F.Cu") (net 13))
 (segment (start 194 71.92) (end 189.38 76.54) (width 0.2) (layer "F.Cu") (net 13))
 (segment (start 160.81 81.62) (end 158 78.81) (width 0.2) (layer "F.Cu") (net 4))
 (segment (start 158 66) (end 160 64) (width 0.2) (layer "F.Cu") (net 4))
 (segment (start 190.54 71.46) (end 189.38 71.46) (width 0.2) (layer "F.Cu") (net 4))
 (segment (start 158 78.81) (end 158 78) (width 0.2) (layer "F.Cu") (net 4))
 (segment (start 160 64) (end 168 64) (width 0.2) (layer "F.Cu") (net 4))
 (segment (start 192 70) (end 190.54 71.46) (width 0.2) (layer "F.Cu") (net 4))
 (segment (start 158 78) (end 158 66) (width 0.2) (layer "F.Cu") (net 4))
 (via (at 168 64) (size 0.6) (drill 0.3) (layers "F.Cu" "B.Cu") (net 4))
 (via (at 192 70) (size 0.6) (drill 0.3) (layers "F.Cu" "B.Cu") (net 4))
 (segment (start 168 64) (end 190 64) (width 0.2) (layer "B.Cu") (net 4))
 (segment (start 192 66) (end 192 70) (width 0.2) (layer "B.Cu") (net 4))
 (segment (start 190 64) (end 192 66) (width 0.2) (layer "B.Cu") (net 4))
 (segment (start 186.08 79.08) (end 189.38 79.08) (width 0.2) (layer "F.Cu") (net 6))
 (segment (start 160.81 74) (end 167 74) (width 0.2) (layer "F.Cu") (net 6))
 (segment (start 184 77) (end 186.08 79.08) (width 0.2) (layer "F.Cu") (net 6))
 (via (at 167 74) (size 0.6) (drill 0.3) (layers "F.Cu" "B.Cu") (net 6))
 (via (at 184 77) (size 0.6) (drill 0.3) (layers "F.Cu" "B.Cu") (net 6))
 (segment (start 167 74) (end 181 74) (width 0.2) (layer "B.Cu") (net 6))
 (segment (start 181 74) (end 184 77) (width 0.2) (layer "B.Cu") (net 6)))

